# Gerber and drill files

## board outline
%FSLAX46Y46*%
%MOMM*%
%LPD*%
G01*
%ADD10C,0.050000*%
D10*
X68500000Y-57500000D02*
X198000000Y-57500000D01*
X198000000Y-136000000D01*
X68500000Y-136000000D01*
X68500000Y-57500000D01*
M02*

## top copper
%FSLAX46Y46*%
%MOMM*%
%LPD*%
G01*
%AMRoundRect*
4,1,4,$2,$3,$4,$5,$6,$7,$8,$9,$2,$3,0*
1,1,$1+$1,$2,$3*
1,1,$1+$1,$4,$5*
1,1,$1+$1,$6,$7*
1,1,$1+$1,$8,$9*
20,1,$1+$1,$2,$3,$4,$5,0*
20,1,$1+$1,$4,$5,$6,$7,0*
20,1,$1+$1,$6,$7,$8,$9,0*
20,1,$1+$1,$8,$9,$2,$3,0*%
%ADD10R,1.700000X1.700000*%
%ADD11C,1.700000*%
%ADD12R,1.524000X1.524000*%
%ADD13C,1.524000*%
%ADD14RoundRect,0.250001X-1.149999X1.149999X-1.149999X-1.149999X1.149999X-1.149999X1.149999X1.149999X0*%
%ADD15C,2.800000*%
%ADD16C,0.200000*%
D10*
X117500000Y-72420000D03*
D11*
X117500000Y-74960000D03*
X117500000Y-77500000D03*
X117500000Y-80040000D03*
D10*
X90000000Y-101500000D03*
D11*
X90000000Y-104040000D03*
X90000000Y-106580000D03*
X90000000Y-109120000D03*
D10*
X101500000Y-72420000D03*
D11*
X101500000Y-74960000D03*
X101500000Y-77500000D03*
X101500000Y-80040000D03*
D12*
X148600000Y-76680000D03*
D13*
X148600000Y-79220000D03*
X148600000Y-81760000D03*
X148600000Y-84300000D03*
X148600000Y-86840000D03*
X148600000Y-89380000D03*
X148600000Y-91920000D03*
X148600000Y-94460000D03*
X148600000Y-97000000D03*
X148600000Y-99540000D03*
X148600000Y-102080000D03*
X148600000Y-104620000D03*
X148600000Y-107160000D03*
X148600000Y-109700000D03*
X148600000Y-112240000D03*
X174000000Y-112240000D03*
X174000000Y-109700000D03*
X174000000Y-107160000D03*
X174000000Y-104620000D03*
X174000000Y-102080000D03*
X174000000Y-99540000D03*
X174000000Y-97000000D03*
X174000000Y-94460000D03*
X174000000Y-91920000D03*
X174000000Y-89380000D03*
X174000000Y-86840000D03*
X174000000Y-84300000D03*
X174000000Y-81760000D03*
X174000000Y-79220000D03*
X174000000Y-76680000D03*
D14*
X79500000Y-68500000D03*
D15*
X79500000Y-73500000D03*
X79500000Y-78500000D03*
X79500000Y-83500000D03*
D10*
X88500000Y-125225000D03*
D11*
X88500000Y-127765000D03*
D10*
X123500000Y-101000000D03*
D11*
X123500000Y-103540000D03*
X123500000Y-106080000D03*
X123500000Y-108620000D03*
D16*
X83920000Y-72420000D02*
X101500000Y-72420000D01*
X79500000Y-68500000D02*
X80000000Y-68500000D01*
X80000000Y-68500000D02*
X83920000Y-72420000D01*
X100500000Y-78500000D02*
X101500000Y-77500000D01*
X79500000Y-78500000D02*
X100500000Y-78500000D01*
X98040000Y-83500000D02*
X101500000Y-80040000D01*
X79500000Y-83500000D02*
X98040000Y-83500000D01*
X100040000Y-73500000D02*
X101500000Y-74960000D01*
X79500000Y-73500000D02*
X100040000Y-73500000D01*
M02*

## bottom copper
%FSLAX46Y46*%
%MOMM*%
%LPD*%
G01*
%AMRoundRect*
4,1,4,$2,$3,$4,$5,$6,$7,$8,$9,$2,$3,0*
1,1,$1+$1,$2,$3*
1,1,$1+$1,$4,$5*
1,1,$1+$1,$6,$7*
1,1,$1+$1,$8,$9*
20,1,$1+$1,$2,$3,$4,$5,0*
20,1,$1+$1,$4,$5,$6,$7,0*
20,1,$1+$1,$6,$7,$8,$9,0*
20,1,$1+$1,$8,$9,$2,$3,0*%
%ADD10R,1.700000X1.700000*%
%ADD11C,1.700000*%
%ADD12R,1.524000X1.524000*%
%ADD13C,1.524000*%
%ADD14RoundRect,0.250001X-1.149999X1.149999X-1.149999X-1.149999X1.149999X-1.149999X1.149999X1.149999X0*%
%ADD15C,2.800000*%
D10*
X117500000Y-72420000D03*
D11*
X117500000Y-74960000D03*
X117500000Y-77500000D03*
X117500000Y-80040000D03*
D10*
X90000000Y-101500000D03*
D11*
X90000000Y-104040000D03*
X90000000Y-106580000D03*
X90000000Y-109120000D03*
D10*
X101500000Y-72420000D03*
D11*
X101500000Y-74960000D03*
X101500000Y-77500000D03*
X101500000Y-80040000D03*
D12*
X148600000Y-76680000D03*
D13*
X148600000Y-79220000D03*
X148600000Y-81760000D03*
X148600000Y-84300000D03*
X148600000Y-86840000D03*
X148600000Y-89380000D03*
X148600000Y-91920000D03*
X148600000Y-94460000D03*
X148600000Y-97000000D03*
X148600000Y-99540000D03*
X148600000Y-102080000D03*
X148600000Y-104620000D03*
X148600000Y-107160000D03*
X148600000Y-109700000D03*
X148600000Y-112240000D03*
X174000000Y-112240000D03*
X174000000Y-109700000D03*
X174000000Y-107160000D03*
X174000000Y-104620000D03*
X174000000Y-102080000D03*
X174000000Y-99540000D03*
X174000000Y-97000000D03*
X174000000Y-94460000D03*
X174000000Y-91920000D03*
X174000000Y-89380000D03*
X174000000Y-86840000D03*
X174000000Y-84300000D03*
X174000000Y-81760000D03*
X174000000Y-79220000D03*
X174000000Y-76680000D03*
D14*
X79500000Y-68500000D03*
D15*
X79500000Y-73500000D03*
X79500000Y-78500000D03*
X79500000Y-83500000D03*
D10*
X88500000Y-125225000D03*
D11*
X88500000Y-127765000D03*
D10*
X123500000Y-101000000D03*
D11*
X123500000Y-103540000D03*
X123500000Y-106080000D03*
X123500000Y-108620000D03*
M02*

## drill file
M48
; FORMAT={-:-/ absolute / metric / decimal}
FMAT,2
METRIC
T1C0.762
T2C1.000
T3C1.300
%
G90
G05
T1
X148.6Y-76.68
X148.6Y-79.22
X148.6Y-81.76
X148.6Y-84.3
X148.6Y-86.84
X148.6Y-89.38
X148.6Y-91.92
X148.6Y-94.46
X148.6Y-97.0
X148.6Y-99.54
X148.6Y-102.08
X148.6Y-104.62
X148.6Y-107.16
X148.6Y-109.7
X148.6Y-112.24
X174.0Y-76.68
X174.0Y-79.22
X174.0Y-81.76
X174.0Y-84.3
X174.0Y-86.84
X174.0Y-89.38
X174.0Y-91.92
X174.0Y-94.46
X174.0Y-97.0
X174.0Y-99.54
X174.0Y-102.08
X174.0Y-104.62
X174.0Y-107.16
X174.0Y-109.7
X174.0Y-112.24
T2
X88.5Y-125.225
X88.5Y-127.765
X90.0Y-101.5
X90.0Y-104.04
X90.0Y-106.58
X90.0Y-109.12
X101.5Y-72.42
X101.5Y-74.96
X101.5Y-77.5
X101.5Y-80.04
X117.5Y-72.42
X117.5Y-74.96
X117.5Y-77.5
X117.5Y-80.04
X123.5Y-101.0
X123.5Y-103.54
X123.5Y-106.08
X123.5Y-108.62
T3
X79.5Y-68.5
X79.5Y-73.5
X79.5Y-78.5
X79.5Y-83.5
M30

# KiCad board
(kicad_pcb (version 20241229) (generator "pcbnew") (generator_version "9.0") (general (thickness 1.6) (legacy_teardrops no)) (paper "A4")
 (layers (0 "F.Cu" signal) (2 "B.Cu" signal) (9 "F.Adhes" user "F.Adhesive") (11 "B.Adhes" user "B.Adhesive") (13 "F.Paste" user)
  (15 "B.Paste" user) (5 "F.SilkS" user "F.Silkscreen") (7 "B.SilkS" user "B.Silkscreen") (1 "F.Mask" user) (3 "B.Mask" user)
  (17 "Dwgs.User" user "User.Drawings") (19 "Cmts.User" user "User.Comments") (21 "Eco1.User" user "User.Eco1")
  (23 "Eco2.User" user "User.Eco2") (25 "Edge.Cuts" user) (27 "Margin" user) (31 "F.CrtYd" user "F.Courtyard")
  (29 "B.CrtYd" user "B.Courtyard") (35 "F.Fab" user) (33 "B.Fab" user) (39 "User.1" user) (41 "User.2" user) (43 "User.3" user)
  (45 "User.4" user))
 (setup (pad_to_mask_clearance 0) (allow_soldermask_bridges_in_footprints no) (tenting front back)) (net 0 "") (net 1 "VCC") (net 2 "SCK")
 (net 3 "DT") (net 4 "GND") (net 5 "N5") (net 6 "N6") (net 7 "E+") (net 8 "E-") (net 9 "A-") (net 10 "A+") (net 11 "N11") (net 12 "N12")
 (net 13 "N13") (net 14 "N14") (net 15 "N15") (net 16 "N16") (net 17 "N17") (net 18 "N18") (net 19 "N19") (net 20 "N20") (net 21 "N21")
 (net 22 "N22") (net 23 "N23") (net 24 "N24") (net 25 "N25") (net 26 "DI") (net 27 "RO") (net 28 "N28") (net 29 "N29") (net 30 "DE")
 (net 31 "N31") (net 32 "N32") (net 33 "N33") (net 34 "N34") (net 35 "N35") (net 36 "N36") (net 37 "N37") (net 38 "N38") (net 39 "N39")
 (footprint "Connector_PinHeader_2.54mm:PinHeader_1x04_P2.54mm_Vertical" (layer "F.Cu") (at 117.5 72.42)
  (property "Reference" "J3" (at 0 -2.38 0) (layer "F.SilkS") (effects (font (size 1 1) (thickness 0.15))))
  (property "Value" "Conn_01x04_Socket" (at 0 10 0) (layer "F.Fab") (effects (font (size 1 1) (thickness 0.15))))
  (pad "1" thru_hole rect (at 0 0) (size 1.7 1.7) (drill 1) (layers "*.Cu" "*.Mask") (remove_unused_layers no) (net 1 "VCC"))
  (pad "2" thru_hole circle (at 0 2.54) (size 1.7 1.7) (drill 1) (layers "*.Cu" "*.Mask") (remove_unused_layers no) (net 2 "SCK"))
  (pad "3" thru_hole circle (at 0 5.08) (size 1.7 1.7) (drill 1) (layers "*.Cu" "*.Mask") (remove_unused_layers no) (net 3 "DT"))
  (pad "4" thru_hole circle (at 0 7.62) (size 1.7 1.7) (drill 1) (layers "*.Cu" "*.Mask") (remove_unused_layers no) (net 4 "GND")))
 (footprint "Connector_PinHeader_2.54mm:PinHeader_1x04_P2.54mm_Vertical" (layer "F.Cu") (at 90 101.5)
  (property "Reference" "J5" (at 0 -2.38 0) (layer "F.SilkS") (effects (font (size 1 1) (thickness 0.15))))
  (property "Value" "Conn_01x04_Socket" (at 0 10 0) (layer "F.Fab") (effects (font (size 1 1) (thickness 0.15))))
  (pad "1" thru_hole rect (at 0 0) (size 1.7 1.7) (drill 1) (layers "*.Cu" "*.Mask") (remove_unused_layers no) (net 1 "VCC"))
  (pad "2" thru_hole circle (at 0 2.54) (size 1.7 1.7) (drill 1) (layers "*.Cu" "*.Mask") (remove_unused_layers no) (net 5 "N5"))
  (pad "3" thru_hole circle (at 0 5.08) (size 1.7 1.7) (drill 1) (layers "*.Cu" "*.Mask") (remove_unused_layers no) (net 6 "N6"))
  (pad "4" thru_hole circle (at 0 7.62) (size 1.7 1.7) (drill 1) (layers "*.Cu" "*.Mask") (remove_unused_layers no) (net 4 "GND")))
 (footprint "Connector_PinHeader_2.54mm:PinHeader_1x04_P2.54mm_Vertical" (layer "F.Cu") (at 101.5 72.42)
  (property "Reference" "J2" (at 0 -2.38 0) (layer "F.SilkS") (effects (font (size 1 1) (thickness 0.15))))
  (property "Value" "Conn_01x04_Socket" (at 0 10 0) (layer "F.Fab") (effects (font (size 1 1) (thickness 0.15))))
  (pad "1" thru_hole rect (at 0 0) (size 1.7 1.7) (drill 1) (layers "*.Cu" "*.Mask") (remove_unused_layers no) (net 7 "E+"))
  (pad "2" thru_hole circle (at 0 2.54) (size 1.7 1.7) (drill 1) (layers "*.Cu" "*.Mask") (remove_unused_layers no) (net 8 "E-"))
  (pad "3" thru_hole circle (at 0 5.08) (size 1.7 1.7) (drill 1) (layers "*.Cu" "*.Mask") (remove_unused_layers no) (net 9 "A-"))
  (pad "4" thru_hole circle (at 0 7.62) (size 1.7 1.7) (drill 1) (layers "*.Cu" "*.Mask") (remove_unused_layers no) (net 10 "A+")))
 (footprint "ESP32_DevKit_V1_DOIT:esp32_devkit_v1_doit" (layer "F.Cu") (at 161.3 76.68)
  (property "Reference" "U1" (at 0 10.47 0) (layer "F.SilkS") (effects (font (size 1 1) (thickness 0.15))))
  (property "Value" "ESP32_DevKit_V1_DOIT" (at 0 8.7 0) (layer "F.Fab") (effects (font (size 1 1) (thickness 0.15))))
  (pad "1" thru_hole rect (at -12.7 0) (size 1.524 1.524) (drill 0.762) (layers "*.Cu" "*.Mask") (remove_unused_layers no) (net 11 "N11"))
  (pad "2" thru_hole circle (at -12.7 2.54) (size 1.524 1.524) (drill 0.762) (layers "*.Cu" "*.Mask") (remove_unused_layers no)
   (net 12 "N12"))
  (pad "3" thru_hole circle (at -12.7 5.08) (size 1.524 1.524) (drill 0.762) (layers "*.Cu" "*.Mask") (remove_unused_layers no)
   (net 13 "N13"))
  (pad "4" thru_hole circle (at -12.7 7.62) (size 1.524 1.524) (drill 0.762) (layers "*.Cu" "*.Mask") (remove_unused_layers no)
   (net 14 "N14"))
  (pad "5" thru_hole circle (at -12.7 10.16) (size 1.524 1.524) (drill 0.762) (layers "*.Cu" "*.Mask") (remove_unused_layers no)
   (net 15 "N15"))
  (pad "6" thru_hole circle (at -12.7 12.7) (size 1.524 1.524) (drill 0.762) (layers "*.Cu" "*.Mask") (remove_unused_layers no)
   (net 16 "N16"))
  (pad "7" thru_hole circle (at -12.7 15.24) (size 1.524 1.524) (drill 0.762) (layers "*.Cu" "*.Mask") (remove_unused_layers no)
   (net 3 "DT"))
  (pad "8" thru_hole circle (at -12.7 17.78) (size 1.524 1.524) (drill 0.762) (layers "*.Cu" "*.Mask") (remove_unused_layers no)
   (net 2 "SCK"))
  (pad "9" thru_hole circle (at -12.7 20.32) (size 1.524 1.524) (drill 0.762) (layers "*.Cu" "*.Mask") (remove_unused_layers no)
   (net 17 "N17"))
  (pad "10" thru_hole circle (at -12.7 22.86) (size 1.524 1.524) (drill 0.762) (layers "*.Cu" "*.Mask") (remove_unused_layers no)
   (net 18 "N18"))
  (pad "11" thru_hole circle (at -12.7 25.4) (size 1.524 1.524) (drill 0.762) (layers "*.Cu" "*.Mask") (remove_unused_layers no)
   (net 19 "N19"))
  (pad "12" thru_hole circle (at -12.7 27.94) (size 1.524 1.524) (drill 0.762) (layers "*.Cu" "*.Mask") (remove_unused_layers no)
   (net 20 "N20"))
  (pad "13" thru_hole circle (at -12.7 30.48) (size 1.524 1.524) (drill 0.762) (layers "*.Cu" "*.Mask") (remove_unused_layers no)
   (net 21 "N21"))
  (pad "14" thru_hole circle (at -12.7 33.02) (size 1.524 1.524) (drill 0.762) (layers "*.Cu" "*.Mask") (remove_unused_layers no)
   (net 4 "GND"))
  (pad "15" thru_hole circle (at -12.7 35.56) (size 1.524 1.524) (drill 0.762) (layers "*.Cu" "*.Mask") (remove_unused_layers no)
   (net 1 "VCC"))
  (pad "16" thru_hole circle (at 12.7 35.56) (size 1.524 1.524) (drill 0.762) (layers "*.Cu" "*.Mask") (remove_unused_layers no)
   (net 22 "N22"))
  (pad "17" thru_hole circle (at 12.7 33.02) (size 1.524 1.524) (drill 0.762) (layers "*.Cu" "*.Mask") (remove_unused_layers no)
   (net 4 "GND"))
  (pad "18" thru_hole circle (at 12.7 30.48) (size 1.524 1.524) (drill 0.762) (layers "*.Cu" "*.Mask") (remove_unused_layers no)
   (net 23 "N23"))
  (pad "19" thru_hole circle (at 12.7 27.94) (size 1.524 1.524) (drill 0.762) (layers "*.Cu" "*.Mask") (remove_unused_layers no)
   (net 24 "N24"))
  (pad "20" thru_hole circle (at 12.7 25.4) (size 1.524 1.524) (drill 0.762) (layers "*.Cu" "*.Mask") (remove_unused_layers no)
   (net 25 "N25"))
  (pad "21" thru_hole circle (at 12.7 22.86) (size 1.524 1.524) (drill 0.762) (layers "*.Cu" "*.Mask") (remove_unused_layers no)
   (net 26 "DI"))
  (pad "22" thru_hole circle (at 12.7 20.32) (size 1.524 1.524) (drill 0.762) (layers "*.Cu" "*.Mask") (remove_unused_layers no)
   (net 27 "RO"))
  (pad "23" thru_hole circle (at 12.7 17.78) (size 1.524 1.524) (drill 0.762) (layers "*.Cu" "*.Mask") (remove_unused_layers no)
   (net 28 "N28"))
  (pad "24" thru_hole circle (at 12.7 15.24) (size 1.524 1.524) (drill 0.762) (layers "*.Cu" "*.Mask") (remove_unused_layers no)
   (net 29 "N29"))
  (pad "25" thru_hole circle (at 12.7 12.7) (size 1.524 1.524) (drill 0.762) (layers "*.Cu" "*.Mask") (remove_unused_layers no)
   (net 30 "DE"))
  (pad "26" thru_hole circle (at 12.7 10.16) (size 1.524 1.524) (drill 0.762) (layers "*.Cu" "*.Mask") (remove_unused_layers no)
   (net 30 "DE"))
  (pad "27" thru_hole circle (at 12.7 7.62) (size 1.524 1.524) (drill 0.762) (layers "*.Cu" "*.Mask") (remove_unused_layers no)
   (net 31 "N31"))
  (pad "28" thru_hole circle (at 12.7 5.08) (size 1.524 1.524) (drill 0.762) (layers "*.Cu" "*.Mask") (remove_unused_layers no)
   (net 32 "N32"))
  (pad "29" thru_hole circle (at 12.7 2.54) (size 1.524 1.524) (drill 0.762) (layers "*.Cu" "*.Mask") (remove_unused_layers no)
   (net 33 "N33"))
  (pad "30" thru_hole circle (at 12.7 0) (size 1.524 1.524) (drill 0.762) (layers "*.Cu" "*.Mask") (remove_unused_layers no) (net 2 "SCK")))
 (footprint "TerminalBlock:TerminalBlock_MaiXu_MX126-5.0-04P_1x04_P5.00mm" (layer "F.Cu") (at 79.5 68.5 -90)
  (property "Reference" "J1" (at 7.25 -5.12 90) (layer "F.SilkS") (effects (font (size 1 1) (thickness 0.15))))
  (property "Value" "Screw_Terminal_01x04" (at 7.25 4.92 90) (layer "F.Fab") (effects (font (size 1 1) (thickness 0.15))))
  (pad "1" thru_hole roundrect (at 0 0 270) (size 2.8 2.8) (drill 1.3) (layers "*.Cu" "*.Mask") (remove_unused_layers no)
   (roundrect_rratio 0.089286) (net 7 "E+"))
  (pad "2" thru_hole circle (at 5 0 270) (size 2.8 2.8) (drill 1.3) (layers "*.Cu" "*.Mask") (remove_unused_layers no) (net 8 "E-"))
  (pad "3" thru_hole circle (at 10 0 270) (size 2.8 2.8) (drill 1.3) (layers "*.Cu" "*.Mask") (remove_unused_layers no) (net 9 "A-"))
  (pad "4" thru_hole circle (at 15 0 270) (size 2.8 2.8) (drill 1.3) (layers "*.Cu" "*.Mask") (remove_unused_layers no) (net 10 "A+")))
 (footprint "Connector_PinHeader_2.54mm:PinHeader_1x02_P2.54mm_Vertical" (layer "F.Cu") (at 88.5 125.225)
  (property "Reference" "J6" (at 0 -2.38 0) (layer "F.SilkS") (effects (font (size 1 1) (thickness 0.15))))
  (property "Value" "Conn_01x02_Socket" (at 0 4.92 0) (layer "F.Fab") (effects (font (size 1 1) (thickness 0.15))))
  (pad "1" thru_hole rect (at 0 0) (size 1.7 1.7) (drill 1) (layers "*.Cu" "*.Mask") (remove_unused_layers no) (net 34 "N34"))
  (pad "2" thru_hole circle (at 0 2.54) (size 1.7 1.7) (drill 1) (layers "*.Cu" "*.Mask") (remove_unused_layers no) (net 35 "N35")))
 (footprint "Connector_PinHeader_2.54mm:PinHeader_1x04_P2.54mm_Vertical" (layer "F.Cu") (at 123.5 101)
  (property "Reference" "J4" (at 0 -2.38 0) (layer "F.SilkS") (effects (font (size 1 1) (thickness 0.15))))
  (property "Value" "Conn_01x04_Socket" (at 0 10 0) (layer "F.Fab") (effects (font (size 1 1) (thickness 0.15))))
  (pad "1" thru_hole rect (at 0 0) (size 1.7 1.7) (drill 1) (layers "*.Cu" "*.Mask") (remove_unused_layers no) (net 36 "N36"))
  (pad "2" thru_hole circle (at 0 2.54) (size 1.7 1.7) (drill 1) (layers "*.Cu" "*.Mask") (remove_unused_layers no) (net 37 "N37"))
  (pad "3" thru_hole circle (at 0 5.08) (size 1.7 1.7) (drill 1) (layers "*.Cu" "*.Mask") (remove_unused_layers no) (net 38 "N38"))
  (pad "4" thru_hole circle (at 0 7.62) (size 1.7 1.7) (drill 1) (layers "*.Cu" "*.Mask") (remove_unused_layers no) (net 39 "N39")))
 (gr_rect (start 68.5 57.5) (end 198 136) (stroke (width 0.05) (type default)) (fill no) (layer "Edge.Cuts"))
 (segment (start 83.92 72.42) (end 101.5 72.42) (width 0.2) (layer "F.Cu") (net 7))
 (segment (start 79.5 68.5) (end 80 68.5) (width 0.2) (layer "F.Cu") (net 7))
 (segment (start 80 68.5) (end 83.92 72.42) (width 0.2) (layer "F.Cu") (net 7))
 (segment (start 100.5 78.5) (end 101.5 77.5) (width 0.2) (layer "F.Cu") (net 9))
 (segment (start 79.5 78.5) (end 100.5 78.5) (width 0.2) (layer "F.Cu") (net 9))
 (segment (start 98.04 83.5) (end 101.5 80.04) (width 0.2) (layer "F.Cu") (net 10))
 (segment (start 79.5 83.5) (end 98.04 83.5) (width 0.2) (layer "F.Cu") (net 10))
 (segment (start 100.04 73.5) (end 101.5 74.96) (width 0.2) (layer "F.Cu") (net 8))
 (segment (start 79.5 73.5) (end 100.04 73.5) (width 0.2) (layer "F.Cu") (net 8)))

